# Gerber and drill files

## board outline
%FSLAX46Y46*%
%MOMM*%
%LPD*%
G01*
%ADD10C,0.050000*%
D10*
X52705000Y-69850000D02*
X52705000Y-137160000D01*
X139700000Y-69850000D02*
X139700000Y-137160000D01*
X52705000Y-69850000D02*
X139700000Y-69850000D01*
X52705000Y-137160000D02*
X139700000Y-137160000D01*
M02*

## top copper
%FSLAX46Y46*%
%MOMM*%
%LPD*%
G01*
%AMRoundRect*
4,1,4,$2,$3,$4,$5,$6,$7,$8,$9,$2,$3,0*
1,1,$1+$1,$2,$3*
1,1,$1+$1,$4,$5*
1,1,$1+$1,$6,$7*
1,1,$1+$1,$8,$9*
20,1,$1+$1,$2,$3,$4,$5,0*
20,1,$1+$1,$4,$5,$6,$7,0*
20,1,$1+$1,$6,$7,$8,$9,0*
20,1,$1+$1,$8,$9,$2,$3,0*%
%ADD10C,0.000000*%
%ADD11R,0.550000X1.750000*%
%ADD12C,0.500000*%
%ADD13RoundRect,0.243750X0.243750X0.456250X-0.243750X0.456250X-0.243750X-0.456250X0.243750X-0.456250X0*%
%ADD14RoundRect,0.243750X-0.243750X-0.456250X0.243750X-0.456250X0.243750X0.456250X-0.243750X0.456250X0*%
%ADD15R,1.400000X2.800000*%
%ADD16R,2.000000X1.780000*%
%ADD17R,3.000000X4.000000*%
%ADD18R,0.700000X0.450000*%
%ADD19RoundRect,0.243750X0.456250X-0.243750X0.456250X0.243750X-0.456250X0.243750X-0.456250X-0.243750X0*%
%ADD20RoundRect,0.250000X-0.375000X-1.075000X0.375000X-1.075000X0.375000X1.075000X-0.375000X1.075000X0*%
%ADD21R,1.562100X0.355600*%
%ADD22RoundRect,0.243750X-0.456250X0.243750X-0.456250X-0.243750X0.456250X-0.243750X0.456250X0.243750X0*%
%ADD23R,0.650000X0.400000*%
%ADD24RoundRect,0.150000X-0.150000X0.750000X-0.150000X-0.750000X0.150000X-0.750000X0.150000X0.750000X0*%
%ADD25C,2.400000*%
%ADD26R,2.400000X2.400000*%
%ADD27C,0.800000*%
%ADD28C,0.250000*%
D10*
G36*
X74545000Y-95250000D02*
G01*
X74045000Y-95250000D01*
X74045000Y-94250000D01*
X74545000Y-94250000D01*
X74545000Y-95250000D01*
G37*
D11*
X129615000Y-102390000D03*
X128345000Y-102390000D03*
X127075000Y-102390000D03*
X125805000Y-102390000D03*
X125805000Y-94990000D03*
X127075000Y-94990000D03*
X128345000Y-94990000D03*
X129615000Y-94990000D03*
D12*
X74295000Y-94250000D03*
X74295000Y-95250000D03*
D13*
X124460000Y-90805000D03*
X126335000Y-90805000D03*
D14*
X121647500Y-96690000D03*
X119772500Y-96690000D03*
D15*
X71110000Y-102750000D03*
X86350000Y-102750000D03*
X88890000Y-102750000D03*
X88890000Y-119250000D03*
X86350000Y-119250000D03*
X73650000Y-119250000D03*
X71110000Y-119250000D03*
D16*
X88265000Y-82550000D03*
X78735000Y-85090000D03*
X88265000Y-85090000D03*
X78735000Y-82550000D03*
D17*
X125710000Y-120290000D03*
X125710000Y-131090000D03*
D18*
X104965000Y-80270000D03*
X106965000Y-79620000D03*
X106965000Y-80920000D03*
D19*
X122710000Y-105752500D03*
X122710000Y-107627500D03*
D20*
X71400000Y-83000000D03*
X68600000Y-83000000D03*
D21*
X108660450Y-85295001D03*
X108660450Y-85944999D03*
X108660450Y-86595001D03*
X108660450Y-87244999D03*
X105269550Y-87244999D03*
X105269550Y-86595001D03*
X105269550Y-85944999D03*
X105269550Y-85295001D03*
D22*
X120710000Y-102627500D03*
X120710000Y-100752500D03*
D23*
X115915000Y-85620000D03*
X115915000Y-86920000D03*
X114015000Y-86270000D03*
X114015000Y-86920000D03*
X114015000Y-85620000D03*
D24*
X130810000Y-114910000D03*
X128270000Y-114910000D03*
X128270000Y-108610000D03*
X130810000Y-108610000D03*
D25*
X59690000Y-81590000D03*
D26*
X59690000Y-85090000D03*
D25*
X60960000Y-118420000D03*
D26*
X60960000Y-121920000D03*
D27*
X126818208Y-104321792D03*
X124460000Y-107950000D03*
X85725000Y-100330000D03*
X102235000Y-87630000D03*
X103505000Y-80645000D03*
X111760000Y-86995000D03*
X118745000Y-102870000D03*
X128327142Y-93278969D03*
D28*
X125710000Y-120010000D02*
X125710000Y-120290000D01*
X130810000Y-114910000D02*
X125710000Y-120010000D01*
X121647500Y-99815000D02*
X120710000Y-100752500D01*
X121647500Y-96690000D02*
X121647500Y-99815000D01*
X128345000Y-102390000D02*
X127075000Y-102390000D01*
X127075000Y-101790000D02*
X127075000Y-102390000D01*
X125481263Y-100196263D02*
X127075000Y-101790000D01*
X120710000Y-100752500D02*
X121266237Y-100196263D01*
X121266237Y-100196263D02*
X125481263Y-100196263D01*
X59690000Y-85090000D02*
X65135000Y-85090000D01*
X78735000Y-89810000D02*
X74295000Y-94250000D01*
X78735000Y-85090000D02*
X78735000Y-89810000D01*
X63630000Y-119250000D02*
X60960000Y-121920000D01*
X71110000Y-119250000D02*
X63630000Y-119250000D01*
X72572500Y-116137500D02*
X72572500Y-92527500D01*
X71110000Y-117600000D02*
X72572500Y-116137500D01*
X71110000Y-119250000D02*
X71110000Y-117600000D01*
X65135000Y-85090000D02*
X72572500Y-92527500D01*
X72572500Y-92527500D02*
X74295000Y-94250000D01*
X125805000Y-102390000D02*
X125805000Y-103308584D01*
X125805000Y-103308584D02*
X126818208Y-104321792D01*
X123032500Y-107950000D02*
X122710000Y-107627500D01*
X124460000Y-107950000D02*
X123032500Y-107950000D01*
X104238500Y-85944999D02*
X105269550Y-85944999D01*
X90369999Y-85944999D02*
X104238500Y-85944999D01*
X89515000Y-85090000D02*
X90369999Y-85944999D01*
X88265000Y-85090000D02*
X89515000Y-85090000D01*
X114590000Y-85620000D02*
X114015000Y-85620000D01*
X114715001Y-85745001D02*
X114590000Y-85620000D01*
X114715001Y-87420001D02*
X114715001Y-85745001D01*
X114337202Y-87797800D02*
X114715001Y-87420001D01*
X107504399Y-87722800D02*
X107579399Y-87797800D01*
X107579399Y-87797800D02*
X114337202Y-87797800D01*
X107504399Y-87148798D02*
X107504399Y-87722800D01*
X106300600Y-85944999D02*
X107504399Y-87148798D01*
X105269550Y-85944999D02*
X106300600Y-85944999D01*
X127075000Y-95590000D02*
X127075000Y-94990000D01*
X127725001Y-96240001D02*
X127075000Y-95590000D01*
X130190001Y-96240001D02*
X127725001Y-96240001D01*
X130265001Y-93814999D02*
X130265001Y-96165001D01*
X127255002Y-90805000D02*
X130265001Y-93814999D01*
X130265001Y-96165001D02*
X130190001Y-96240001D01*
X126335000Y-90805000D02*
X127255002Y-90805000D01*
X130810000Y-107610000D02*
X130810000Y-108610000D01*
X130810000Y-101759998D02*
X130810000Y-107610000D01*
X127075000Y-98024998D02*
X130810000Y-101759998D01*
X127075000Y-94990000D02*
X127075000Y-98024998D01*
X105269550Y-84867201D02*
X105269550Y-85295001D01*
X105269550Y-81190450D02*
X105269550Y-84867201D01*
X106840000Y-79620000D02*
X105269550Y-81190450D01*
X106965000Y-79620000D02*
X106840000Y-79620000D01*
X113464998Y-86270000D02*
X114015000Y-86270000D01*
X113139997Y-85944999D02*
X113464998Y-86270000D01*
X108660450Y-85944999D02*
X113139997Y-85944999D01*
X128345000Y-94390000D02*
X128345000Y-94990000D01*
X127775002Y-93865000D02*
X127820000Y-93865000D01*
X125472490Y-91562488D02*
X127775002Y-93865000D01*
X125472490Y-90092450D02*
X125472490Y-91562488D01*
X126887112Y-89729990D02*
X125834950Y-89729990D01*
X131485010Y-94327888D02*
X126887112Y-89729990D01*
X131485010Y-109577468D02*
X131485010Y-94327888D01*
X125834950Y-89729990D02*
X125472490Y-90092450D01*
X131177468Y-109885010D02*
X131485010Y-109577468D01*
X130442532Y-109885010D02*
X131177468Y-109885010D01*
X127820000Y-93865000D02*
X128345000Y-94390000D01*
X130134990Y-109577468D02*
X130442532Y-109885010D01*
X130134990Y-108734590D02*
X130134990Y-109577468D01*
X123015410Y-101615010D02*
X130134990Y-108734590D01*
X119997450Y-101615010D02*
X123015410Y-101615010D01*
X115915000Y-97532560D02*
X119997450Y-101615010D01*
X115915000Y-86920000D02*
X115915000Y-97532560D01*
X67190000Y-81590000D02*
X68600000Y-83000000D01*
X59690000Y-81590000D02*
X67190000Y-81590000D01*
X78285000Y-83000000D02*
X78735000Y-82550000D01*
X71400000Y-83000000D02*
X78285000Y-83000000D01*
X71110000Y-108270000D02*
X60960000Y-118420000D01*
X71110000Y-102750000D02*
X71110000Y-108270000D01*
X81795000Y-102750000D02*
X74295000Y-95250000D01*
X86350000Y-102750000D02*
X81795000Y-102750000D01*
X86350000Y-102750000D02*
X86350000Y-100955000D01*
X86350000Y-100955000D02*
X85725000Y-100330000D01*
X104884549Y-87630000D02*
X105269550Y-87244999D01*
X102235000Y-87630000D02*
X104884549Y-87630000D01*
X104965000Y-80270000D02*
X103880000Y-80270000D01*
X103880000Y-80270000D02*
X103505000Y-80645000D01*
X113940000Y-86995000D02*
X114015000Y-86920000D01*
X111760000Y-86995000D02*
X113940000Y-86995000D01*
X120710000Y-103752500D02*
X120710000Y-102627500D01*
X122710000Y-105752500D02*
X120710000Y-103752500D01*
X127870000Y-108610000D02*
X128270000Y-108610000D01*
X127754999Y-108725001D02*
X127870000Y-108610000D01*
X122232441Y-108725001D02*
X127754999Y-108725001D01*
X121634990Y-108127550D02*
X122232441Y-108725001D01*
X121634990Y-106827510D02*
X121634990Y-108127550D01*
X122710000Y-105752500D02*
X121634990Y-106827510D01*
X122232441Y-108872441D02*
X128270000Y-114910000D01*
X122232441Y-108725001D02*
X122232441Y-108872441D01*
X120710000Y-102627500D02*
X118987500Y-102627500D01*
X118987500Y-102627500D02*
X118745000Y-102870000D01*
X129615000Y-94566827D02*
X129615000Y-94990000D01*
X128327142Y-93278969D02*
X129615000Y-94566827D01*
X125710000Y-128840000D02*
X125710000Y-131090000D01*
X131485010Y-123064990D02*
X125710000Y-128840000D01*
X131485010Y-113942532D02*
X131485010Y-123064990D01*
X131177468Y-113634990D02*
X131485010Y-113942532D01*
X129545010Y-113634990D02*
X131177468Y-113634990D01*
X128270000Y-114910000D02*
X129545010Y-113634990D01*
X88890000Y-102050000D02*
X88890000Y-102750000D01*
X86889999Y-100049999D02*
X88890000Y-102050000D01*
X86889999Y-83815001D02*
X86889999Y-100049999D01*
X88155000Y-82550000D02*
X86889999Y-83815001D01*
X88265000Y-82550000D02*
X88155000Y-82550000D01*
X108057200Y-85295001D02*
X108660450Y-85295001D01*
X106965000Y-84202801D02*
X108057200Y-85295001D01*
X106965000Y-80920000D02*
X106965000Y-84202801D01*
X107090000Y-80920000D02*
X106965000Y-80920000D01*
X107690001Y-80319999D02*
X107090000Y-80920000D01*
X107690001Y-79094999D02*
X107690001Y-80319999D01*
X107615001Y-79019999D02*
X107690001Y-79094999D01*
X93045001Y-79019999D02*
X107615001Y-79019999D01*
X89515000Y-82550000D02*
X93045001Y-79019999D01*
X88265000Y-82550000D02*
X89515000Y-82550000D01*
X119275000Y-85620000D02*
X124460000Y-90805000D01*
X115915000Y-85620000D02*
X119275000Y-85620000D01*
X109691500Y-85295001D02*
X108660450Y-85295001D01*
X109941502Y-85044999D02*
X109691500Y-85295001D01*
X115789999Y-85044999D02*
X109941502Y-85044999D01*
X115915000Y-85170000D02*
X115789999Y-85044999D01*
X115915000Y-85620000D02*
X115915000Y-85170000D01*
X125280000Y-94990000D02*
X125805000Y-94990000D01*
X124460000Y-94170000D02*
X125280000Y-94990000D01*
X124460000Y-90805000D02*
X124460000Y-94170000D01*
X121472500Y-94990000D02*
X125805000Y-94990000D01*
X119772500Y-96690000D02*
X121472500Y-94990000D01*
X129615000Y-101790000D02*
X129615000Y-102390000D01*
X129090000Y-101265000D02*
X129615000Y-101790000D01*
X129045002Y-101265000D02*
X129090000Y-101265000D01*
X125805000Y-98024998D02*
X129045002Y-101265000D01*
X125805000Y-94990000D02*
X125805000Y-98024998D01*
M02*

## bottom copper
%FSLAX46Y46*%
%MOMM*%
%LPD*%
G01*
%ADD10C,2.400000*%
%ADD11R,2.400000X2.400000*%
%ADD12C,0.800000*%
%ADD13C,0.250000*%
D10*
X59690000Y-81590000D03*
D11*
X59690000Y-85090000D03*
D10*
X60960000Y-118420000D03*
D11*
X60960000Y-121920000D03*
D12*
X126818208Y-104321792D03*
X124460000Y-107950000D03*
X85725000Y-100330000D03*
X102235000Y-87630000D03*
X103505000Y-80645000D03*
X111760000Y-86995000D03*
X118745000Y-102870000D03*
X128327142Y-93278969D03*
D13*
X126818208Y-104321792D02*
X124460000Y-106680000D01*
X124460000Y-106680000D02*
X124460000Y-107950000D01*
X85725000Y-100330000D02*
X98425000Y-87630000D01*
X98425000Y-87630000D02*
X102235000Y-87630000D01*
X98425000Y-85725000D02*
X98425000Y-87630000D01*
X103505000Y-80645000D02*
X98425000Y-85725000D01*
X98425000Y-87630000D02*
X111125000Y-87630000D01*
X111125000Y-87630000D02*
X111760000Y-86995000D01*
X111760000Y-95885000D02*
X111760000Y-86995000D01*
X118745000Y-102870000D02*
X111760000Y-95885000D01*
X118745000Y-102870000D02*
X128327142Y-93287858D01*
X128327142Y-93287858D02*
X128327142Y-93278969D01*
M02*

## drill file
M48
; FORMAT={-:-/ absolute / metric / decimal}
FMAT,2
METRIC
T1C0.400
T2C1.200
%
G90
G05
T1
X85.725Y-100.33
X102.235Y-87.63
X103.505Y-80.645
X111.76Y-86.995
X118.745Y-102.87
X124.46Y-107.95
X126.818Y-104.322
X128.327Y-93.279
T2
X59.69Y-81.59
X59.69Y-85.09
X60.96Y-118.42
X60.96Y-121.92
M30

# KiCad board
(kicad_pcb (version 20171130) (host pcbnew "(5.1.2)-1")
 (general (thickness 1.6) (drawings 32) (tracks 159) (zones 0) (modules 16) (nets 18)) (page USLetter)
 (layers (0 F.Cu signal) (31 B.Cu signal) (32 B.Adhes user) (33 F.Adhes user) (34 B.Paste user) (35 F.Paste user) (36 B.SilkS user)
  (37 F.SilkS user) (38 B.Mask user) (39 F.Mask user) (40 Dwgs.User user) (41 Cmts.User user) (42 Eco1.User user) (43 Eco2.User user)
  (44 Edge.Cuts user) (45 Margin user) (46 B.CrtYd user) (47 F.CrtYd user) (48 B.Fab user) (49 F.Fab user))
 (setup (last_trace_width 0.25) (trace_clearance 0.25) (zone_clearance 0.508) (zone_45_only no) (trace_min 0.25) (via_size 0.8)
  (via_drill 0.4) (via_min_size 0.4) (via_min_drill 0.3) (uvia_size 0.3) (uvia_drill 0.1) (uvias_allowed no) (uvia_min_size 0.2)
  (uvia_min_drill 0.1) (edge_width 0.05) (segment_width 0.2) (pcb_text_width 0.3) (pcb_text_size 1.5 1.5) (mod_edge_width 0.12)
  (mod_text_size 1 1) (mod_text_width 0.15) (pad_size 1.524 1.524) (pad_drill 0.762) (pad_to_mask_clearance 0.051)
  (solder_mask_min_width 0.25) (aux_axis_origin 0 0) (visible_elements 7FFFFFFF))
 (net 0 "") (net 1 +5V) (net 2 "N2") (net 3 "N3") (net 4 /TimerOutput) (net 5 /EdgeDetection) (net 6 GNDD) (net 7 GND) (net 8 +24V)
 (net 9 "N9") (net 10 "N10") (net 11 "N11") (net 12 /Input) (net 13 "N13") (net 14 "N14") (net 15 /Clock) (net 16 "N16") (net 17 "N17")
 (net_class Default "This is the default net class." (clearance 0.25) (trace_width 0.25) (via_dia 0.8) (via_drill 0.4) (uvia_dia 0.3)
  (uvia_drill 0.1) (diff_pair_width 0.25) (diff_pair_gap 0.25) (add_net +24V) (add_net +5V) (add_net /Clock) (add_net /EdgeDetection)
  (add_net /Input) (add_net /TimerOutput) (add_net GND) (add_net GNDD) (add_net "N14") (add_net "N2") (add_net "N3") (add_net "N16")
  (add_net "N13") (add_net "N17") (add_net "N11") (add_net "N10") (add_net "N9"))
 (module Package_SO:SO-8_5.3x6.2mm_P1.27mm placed (layer F.Cu) (at 127.71 98.69 270)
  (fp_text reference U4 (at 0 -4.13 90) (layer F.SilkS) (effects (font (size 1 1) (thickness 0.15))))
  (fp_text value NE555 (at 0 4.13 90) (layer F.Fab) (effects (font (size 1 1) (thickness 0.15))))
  (pad 8 smd rect (at 3.7 -1.905 270) (size 1.75 0.55) (layers F.Cu F.Paste F.Mask) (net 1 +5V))
  (pad 7 smd rect (at 3.7 -0.635 270) (size 1.75 0.55) (layers F.Cu F.Paste F.Mask) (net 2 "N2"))
  (pad 6 smd rect (at 3.7 0.635 270) (size 1.75 0.55) (layers F.Cu F.Paste F.Mask) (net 2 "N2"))
  (pad 5 smd rect (at 3.7 1.905 270) (size 1.75 0.55) (layers F.Cu F.Paste F.Mask) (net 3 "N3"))
  (pad 4 smd rect (at -3.7 1.905 270) (size 1.75 0.55) (layers F.Cu F.Paste F.Mask) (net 1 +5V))
  (pad 3 smd rect (at -3.7 0.635 270) (size 1.75 0.55) (layers F.Cu F.Paste F.Mask) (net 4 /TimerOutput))
  (pad 2 smd rect (at -3.7 -0.635 270) (size 1.75 0.55) (layers F.Cu F.Paste F.Mask) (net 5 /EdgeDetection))
  (pad 1 smd rect (at -3.7 -1.905 270) (size 1.75 0.55) (layers F.Cu F.Paste F.Mask) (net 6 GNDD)))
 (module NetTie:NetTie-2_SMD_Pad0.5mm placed (layer F.Cu) (at 74.295 94.75 90)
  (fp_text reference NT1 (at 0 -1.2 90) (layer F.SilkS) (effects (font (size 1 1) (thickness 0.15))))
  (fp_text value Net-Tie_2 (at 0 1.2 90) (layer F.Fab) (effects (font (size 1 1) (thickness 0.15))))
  (fp_poly (pts (xy -0.5 -0.25) (xy 0.5 -0.25) (xy 0.5 0.25) (xy -0.5 0.25)) (layer F.Cu) (width 0))
  (pad 2 smd circle (at 0.5 0 90) (size 0.5 0.5) (layers F.Cu) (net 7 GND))
  (pad 1 smd circle (at -0.5 0 90) (size 0.5 0.5) (layers F.Cu) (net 6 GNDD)))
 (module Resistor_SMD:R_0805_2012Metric (layer F.Cu) (at 125.3975 90.805 180)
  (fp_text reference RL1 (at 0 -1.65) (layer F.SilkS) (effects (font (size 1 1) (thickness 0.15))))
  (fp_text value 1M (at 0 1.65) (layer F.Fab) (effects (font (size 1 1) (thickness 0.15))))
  (pad 2 smd roundrect (at 0.9375 0 180) (size 0.975 1.4) (layers F.Cu F.Paste F.Mask) (roundrect_rratio 0.25) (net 1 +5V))
  (pad 1 smd roundrect (at -0.9375 0 180) (size 0.975 1.4) (layers F.Cu F.Paste F.Mask) (roundrect_rratio 0.25) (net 4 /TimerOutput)))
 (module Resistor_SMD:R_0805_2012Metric (layer F.Cu) (at 120.71 96.69)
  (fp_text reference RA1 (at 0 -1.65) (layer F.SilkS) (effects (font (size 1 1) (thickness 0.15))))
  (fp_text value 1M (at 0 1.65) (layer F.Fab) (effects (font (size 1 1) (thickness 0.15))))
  (pad 2 smd roundrect (at 0.9375 0) (size 0.975 1.4) (layers F.Cu F.Paste F.Mask) (roundrect_rratio 0.25) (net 2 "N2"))
  (pad 1 smd roundrect (at -0.9375 0) (size 0.975 1.4) (layers F.Cu F.Paste F.Mask) (roundrect_rratio 0.25) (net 1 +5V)))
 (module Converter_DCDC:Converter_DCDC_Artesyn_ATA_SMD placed (layer F.Cu) (at 80 111 90)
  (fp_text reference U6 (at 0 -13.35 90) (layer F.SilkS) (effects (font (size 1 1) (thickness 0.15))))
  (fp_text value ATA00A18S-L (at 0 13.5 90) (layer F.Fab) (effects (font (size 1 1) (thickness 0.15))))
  (pad 16 smd rect (at 8.25 -8.89 90) (size 2.8 1.4) (layers F.Cu F.Paste F.Mask) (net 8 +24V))
  (pad 10 smd rect (at 8.25 6.35 90) (size 2.8 1.4) (layers F.Cu F.Paste F.Mask) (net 6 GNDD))
  (pad 9 smd rect (at 8.25 8.89 90) (size 2.8 1.4) (layers F.Cu F.Paste F.Mask) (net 1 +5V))
  (pad 8 smd rect (at -8.25 8.89 90) (size 2.8 1.4) (layers F.Cu F.Paste F.Mask) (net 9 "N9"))
  (pad 7 smd rect (at -8.25 6.35 90) (size 2.8 1.4) (layers F.Cu F.Paste F.Mask) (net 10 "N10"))
  (pad 2 smd rect (at -8.25 -6.35 90) (size 2.8 1.4) (layers F.Cu F.Paste F.Mask) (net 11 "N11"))
  (pad 1 smd rect (at -8.25 -8.89 90) (size 2.8 1.4) (layers F.Cu F.Paste F.Mask) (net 7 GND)))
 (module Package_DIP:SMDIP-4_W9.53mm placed (layer F.Cu) (at 83.5 83.82)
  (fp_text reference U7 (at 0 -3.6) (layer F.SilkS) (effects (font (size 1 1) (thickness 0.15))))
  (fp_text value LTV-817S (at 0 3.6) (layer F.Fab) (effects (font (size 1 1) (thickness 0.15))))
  (pad 4 smd rect (at 4.765 -1.27) (size 2 1.78) (layers F.Cu F.Paste F.Mask) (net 1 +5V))
  (pad 2 smd rect (at -4.765 1.27) (size 2 1.78) (layers F.Cu F.Paste F.Mask) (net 7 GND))
  (pad 3 smd rect (at 4.765 1.27) (size 2 1.78) (layers F.Cu F.Paste F.Mask) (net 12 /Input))
  (pad 1 smd rect (at -4.765 -1.27) (size 2 1.78) (layers F.Cu F.Paste F.Mask) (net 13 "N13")))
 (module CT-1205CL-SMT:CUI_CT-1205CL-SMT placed (layer F.Cu) (at 125.71 125.69 90)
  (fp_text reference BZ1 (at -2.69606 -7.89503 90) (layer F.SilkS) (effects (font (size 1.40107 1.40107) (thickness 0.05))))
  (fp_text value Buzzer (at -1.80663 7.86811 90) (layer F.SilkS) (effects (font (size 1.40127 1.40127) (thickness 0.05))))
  (pad 1 smd rect (at 5.4 0 90) (size 4 3) (layers F.Cu F.Paste F.Mask) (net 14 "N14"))
  (pad 2 smd rect (at -5.4 0 90) (size 4 3) (layers F.Cu F.Paste F.Mask) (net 6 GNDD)))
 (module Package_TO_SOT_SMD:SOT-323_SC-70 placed (layer F.Cu) (at 105.965 80.27 180)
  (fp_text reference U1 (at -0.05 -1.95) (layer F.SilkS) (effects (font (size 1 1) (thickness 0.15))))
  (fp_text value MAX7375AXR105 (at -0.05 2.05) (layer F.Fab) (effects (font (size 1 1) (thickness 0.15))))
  (pad 3 smd rect (at 1 0 90) (size 0.45 0.7) (layers F.Cu F.Paste F.Mask) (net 6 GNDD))
  (pad 2 smd rect (at -1 0.65 90) (size 0.45 0.7) (layers F.Cu F.Paste F.Mask) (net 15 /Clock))
  (pad 1 smd rect (at -1 -0.65 90) (size 0.45 0.7) (layers F.Cu F.Paste F.Mask) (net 1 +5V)))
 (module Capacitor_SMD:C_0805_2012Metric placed (layer F.Cu) (at 122.71 106.69 90)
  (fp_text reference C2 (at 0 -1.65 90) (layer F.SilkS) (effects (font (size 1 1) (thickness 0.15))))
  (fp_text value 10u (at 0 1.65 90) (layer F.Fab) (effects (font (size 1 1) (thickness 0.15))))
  (pad 2 smd roundrect (at 0.9375 0 90) (size 0.975 1.4) (layers F.Cu F.Paste F.Mask) (roundrect_rratio 0.25) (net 6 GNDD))
  (pad 1 smd roundrect (at -0.9375 0 90) (size 0.975 1.4) (layers F.Cu F.Paste F.Mask) (roundrect_rratio 0.25) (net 3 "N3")))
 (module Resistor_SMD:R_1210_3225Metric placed (layer F.Cu) (at 70 83)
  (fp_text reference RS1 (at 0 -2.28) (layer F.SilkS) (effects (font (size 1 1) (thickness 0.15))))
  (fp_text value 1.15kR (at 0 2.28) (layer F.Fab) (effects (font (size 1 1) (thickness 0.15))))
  (pad 2 smd roundrect (at 1.4 0) (size 1.25 2.65) (layers F.Cu F.Paste F.Mask) (roundrect_rratio 0.2) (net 13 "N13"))
  (pad 1 smd roundrect (at -1.4 0) (size 1.25 2.65) (layers F.Cu F.Paste F.Mask) (roundrect_rratio 0.2) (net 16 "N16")))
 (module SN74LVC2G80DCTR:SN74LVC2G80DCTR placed (layer F.Cu) (at 106.965 86.27)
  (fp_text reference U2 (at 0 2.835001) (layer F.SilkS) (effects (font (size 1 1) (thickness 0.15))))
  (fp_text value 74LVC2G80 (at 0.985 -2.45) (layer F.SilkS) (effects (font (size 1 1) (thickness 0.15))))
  (pad 8 smd rect (at 1.69545 -0.974999) (size 1.5621 0.3556) (layers F.Cu F.Paste F.Mask) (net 1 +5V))
  (pad 7 smd rect (at 1.69545 -0.325001) (size 1.5621 0.3556) (layers F.Cu F.Paste F.Mask) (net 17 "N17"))
  (pad 6 smd rect (at 1.69545 0.325001) (size 1.5621 0.3556) (layers F.Cu F.Paste F.Mask))
  (pad 5 smd rect (at 1.69545 0.974999) (size 1.5621 0.3556) (layers F.Cu F.Paste F.Mask))
  (pad 4 smd rect (at -1.69545 0.974999) (size 1.5621 0.3556) (layers F.Cu F.Paste F.Mask) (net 6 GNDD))
  (pad 3 smd rect (at -1.69545 0.325001) (size 1.5621 0.3556) (layers F.Cu F.Paste F.Mask))
  (pad 2 smd rect (at -1.69545 -0.325001) (size 1.5621 0.3556) (layers F.Cu F.Paste F.Mask) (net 12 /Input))
  (pad 1 smd rect (at -1.69545 -0.974999) (size 1.5621 0.3556) (layers F.Cu F.Paste F.Mask) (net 15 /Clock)))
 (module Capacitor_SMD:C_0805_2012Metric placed (layer F.Cu) (at 120.71 101.69 270)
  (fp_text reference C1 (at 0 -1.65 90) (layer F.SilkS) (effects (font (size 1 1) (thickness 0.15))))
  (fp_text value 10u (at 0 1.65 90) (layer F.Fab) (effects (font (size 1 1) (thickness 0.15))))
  (pad 2 smd roundrect (at 0.9375 0 270) (size 0.975 1.4) (layers F.Cu F.Paste F.Mask) (roundrect_rratio 0.25) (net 6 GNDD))
  (pad 1 smd roundrect (at -0.9375 0 270) (size 0.975 1.4) (layers F.Cu F.Paste F.Mask) (roundrect_rratio 0.25) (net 2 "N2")))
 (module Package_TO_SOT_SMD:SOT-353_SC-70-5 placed (layer F.Cu) (at 114.965 86.27)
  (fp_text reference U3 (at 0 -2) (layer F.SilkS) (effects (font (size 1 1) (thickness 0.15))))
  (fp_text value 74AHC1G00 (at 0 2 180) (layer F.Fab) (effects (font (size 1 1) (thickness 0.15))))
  (pad 5 smd rect (at 0.95 -0.65) (size 0.65 0.4) (layers F.Cu F.Paste F.Mask) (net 1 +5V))
  (pad 4 smd rect (at 0.95 0.65) (size 0.65 0.4) (layers F.Cu F.Paste F.Mask) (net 5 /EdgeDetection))
  (pad 2 smd rect (at -0.95 0) (size 0.65 0.4) (layers F.Cu F.Paste F.Mask) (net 17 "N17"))
  (pad 3 smd rect (at -0.95 0.65) (size 0.65 0.4) (layers F.Cu F.Paste F.Mask) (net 6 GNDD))
  (pad 1 smd rect (at -0.95 -0.65) (size 0.65 0.4) (layers F.Cu F.Paste F.Mask) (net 12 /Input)))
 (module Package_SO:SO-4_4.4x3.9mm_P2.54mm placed (layer F.Cu) (at 129.54 111.76 270)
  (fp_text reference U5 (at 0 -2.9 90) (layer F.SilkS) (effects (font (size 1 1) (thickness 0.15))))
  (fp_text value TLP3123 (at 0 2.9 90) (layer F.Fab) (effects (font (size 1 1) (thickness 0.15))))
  (pad 4 smd roundrect (at 3.15 -1.27 270) (size 1.8 0.6) (layers F.Cu F.Paste F.Mask) (roundrect_rratio 0.25) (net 14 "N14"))
  (pad 3 smd roundrect (at 3.15 1.27 270) (size 1.8 0.6) (layers F.Cu F.Paste F.Mask) (roundrect_rratio 0.25) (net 6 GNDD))
  (pad 2 smd roundrect (at -3.15 1.27 270) (size 1.8 0.6) (layers F.Cu F.Paste F.Mask) (roundrect_rratio 0.25) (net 6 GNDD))
  (pad 1 smd roundrect (at -3.15 -1.27 270) (size 1.8 0.6) (layers F.Cu F.Paste F.Mask) (roundrect_rratio 0.25) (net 4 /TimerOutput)))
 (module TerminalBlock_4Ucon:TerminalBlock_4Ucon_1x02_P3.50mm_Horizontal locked (layer F.Cu) (at 59.69 85.09 90)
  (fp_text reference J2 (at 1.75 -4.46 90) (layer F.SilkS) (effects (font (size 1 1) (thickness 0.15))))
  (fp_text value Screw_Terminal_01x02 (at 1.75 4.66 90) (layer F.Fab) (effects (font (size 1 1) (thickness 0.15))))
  (pad 2 thru_hole circle (at 3.5 0 90) (size 2.4 2.4) (drill 1.2) (layers *.Cu *.Mask) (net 16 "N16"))
  (pad 1 thru_hole rect (at 0 0 90) (size 2.4 2.4) (drill 1.2) (layers *.Cu *.Mask) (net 7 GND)))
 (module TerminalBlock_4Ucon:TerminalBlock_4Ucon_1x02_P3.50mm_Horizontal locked (layer F.Cu) (at 60.96 121.92 90)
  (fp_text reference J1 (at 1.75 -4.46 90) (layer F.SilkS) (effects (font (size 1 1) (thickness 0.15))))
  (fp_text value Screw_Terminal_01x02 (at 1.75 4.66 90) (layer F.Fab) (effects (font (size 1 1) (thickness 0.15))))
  (pad 2 thru_hole circle (at 3.5 0 90) (size 2.4 2.4) (drill 1.2) (layers *.Cu *.Mask) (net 8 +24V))
  (pad 1 thru_hole rect (at 0 0 90) (size 2.4 2.4) (drill 1.2) (layers *.Cu *.Mask) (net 7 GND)))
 (gr_line (start 52.705 69.85) (end 52.705 137.16) (layer Edge.Cuts) (width 0.05))
 (gr_line (start 139.7 69.85) (end 139.7 137.16) (layer Edge.Cuts) (width 0.05))
 (gr_line (start 52.705 69.85) (end 139.7 69.85) (layer Edge.Cuts) (width 0.05))
 (gr_line (start 52.705 137.16) (end 139.7 137.16) (layer Edge.Cuts) (width 0.05))
 (segment (start 125.71 120.01) (end 125.71 120.29) (width 0.25) (layer F.Cu) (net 14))
 (segment (start 130.81 114.91) (end 125.71 120.01) (width 0.25) (layer F.Cu) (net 14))
 (segment (start 121.6475 99.815) (end 120.71 100.7525) (width 0.25) (layer F.Cu) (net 2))
 (segment (start 121.6475 96.69) (end 121.6475 99.815) (width 0.25) (layer F.Cu) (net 2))
 (segment (start 128.345 102.39) (end 127.075 102.39) (width 0.25) (layer F.Cu) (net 2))
 (segment (start 127.075 101.79) (end 127.075 102.39) (width 0.25) (layer F.Cu) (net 2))
 (segment (start 125.481263 100.196263) (end 127.075 101.79) (width 0.25) (layer F.Cu) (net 2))
 (segment (start 120.71 100.7525) (end 121.266237 100.196263) (width 0.25) (layer F.Cu) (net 2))
 (segment (start 121.266237 100.196263) (end 125.481263 100.196263) (width 0.25) (layer F.Cu) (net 2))
 (segment (start 59.69 85.09) (end 65.135 85.09) (width 0.25) (layer F.Cu) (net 7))
 (segment (start 78.735 89.81) (end 74.295 94.25) (width 0.25) (layer F.Cu) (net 7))
 (segment (start 78.735 85.09) (end 78.735 89.81) (width 0.25) (layer F.Cu) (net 7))
 (segment (start 63.63 119.25) (end 60.96 121.92) (width 0.25) (layer F.Cu) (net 7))
 (segment (start 71.11 119.25) (end 63.63 119.25) (width 0.25) (layer F.Cu) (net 7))
 (segment (start 72.5725 116.1375) (end 72.5725 92.5275) (width 0.25) (layer F.Cu) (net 7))
 (segment (start 71.11 117.6) (end 72.5725 116.1375) (width 0.25) (layer F.Cu) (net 7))
 (segment (start 71.11 119.25) (end 71.11 117.6) (width 0.25) (layer F.Cu) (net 7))
 (segment (start 65.135 85.09) (end 72.5725 92.5275) (width 0.25) (layer F.Cu) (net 7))
 (segment (start 72.5725 92.5275) (end 74.295 94.25) (width 0.25) (layer F.Cu) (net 7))
 (via (at 126.818208 104.321792) (size 0.8) (drill 0.4) (layers F.Cu B.Cu) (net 3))
 (segment (start 125.805 102.39) (end 125.805 103.308584) (width 0.25) (layer F.Cu) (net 3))
 (segment (start 125.805 103.308584) (end 126.818208 104.321792) (width 0.25) (layer F.Cu) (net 3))
 (via (at 124.46 107.95) (size 0.8) (drill 0.4) (layers F.Cu B.Cu) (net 3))
 (segment (start 126.818208 104.321792) (end 124.46 106.68) (width 0.25) (layer B.Cu) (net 3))
 (segment (start 124.46 106.68) (end 124.46 107.95) (width 0.25) (layer B.Cu) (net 3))
 (segment (start 123.0325 107.95) (end 122.71 107.6275) (width 0.25) (layer F.Cu) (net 3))
 (segment (start 124.46 107.95) (end 123.0325 107.95) (width 0.25) (layer F.Cu) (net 3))
 (segment (start 104.2385 85.944999) (end 105.26955 85.944999) (width 0.25) (layer F.Cu) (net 12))
 (segment (start 90.369999 85.944999) (end 104.2385 85.944999) (width 0.25) (layer F.Cu) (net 12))
 (segment (start 89.515 85.09) (end 90.369999 85.944999) (width 0.25) (layer F.Cu) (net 12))
 (segment (start 88.265 85.09) (end 89.515 85.09) (width 0.25) (layer F.Cu) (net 12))
 (segment (start 114.59 85.62) (end 114.015 85.62) (width 0.25) (layer F.Cu) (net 12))
 (segment (start 114.715001 85.745001) (end 114.59 85.62) (width 0.25) (layer F.Cu) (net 12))
 (segment (start 114.715001 87.420001) (end 114.715001 85.745001) (width 0.25) (layer F.Cu) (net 12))
 (segment (start 114.337202 87.7978) (end 114.715001 87.420001) (width 0.25) (layer F.Cu) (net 12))
 (segment (start 107.504399 87.7228) (end 107.579399 87.7978) (width 0.25) (layer F.Cu) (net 12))
 (segment (start 107.579399 87.7978) (end 114.337202 87.7978) (width 0.25) (layer F.Cu) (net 12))
 (segment (start 107.504399 87.148798) (end 107.504399 87.7228) (width 0.25) (layer F.Cu) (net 12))
 (segment (start 106.3006 85.944999) (end 107.504399 87.148798) (width 0.25) (layer F.Cu) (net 12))
 (segment (start 105.26955 85.944999) (end 106.3006 85.944999) (width 0.25) (layer F.Cu) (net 12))
 (segment (start 127.075 95.59) (end 127.075 94.99) (width 0.25) (layer F.Cu) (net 4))
 (segment (start 127.725001 96.240001) (end 127.075 95.59) (width 0.25) (layer F.Cu) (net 4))
 (segment (start 130.190001 96.240001) (end 127.725001 96.240001) (width 0.25) (layer F.Cu) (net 4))
 (segment (start 130.265001 93.814999) (end 130.265001 96.165001) (width 0.25) (layer F.Cu) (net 4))
 (segment (start 127.255002 90.805) (end 130.265001 93.814999) (width 0.25) (layer F.Cu) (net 4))
 (segment (start 130.265001 96.165001) (end 130.190001 96.240001) (width 0.25) (layer F.Cu) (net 4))
 (segment (start 126.335 90.805) (end 127.255002 90.805) (width 0.25) (layer F.Cu) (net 4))
 (segment (start 130.81 107.61) (end 130.81 108.61) (width 0.25) (layer F.Cu) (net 4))
 (segment (start 130.81 101.759998) (end 130.81 107.61) (width 0.25) (layer F.Cu) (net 4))
 (segment (start 127.075 98.024998) (end 130.81 101.759998) (width 0.25) (layer F.Cu) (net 4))
 (segment (start 127.075 94.99) (end 127.075 98.024998) (width 0.25) (layer F.Cu) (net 4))
 (segment (start 105.26955 84.867201) (end 105.26955 85.295001) (width 0.25) (layer F.Cu) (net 15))
 (segment (start 105.26955 81.19045) (end 105.26955 84.867201) (width 0.25) (layer F.Cu) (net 15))
 (segment (start 106.84 79.62) (end 105.26955 81.19045) (width 0.25) (layer F.Cu) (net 15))
 (segment (start 106.965 79.62) (end 106.84 79.62) (width 0.25) (layer F.Cu) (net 15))
 (segment (start 113.464998 86.27) (end 114.015 86.27) (width 0.25) (layer F.Cu) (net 17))
 (segment (start 113.139997 85.944999) (end 113.464998 86.27) (width 0.25) (layer F.Cu) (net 17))
 (segment (start 108.66045 85.944999) (end 113.139997 85.944999) (width 0.25) (layer F.Cu) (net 17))
 (segment (start 128.345 94.39) (end 128.345 94.99) (width 0.25) (layer F.Cu) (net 5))
 (segment (start 127.775002 93.865) (end 127.82 93.865) (width 0.25) (layer F.Cu) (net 5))
 (segment (start 125.47249 91.562488) (end 127.775002 93.865) (width 0.25) (layer F.Cu) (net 5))
 (segment (start 125.47249 90.09245) (end 125.47249 91.562488) (width 0.25) (layer F.Cu) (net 5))
 (segment (start 126.887112 89.72999) (end 125.83495 89.72999) (width 0.25) (layer F.Cu) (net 5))
 (segment (start 131.48501 94.327888) (end 126.887112 89.72999) (width 0.25) (layer F.Cu) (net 5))
 (segment (start 131.48501 109.577468) (end 131.48501 94.327888) (width 0.25) (layer F.Cu) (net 5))
 (segment (start 125.83495 89.72999) (end 125.47249 90.09245) (width 0.25) (layer F.Cu) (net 5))
 (segment (start 131.177468 109.88501) (end 131.48501 109.577468) (width 0.25) (layer F.Cu) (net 5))
 (segment (start 130.442532 109.88501) (end 131.177468 109.88501) (width 0.25) (layer F.Cu) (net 5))
 (segment (start 127.82 93.865) (end 128.345 94.39) (width 0.25) (layer F.Cu) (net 5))
 (segment (start 130.13499 109.577468) (end 130.442532 109.88501) (width 0.25) (layer F.Cu) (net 5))
 (segment (start 130.13499 108.73459) (end 130.13499 109.577468) (width 0.25) (layer F.Cu) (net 5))
 (segment (start 123.01541 101.61501) (end 130.13499 108.73459) (width 0.25) (layer F.Cu) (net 5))
 (segment (start 119.99745 101.61501) (end 123.01541 101.61501) (width 0.25) (layer F.Cu) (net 5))
 (segment (start 115.915 97.53256) (end 119.99745 101.61501) (width 0.25) (layer F.Cu) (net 5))
 (segment (start 115.915 86.92) (end 115.915 97.53256) (width 0.25) (layer F.Cu) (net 5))
 (segment (start 67.19 81.59) (end 68.6 83) (width 0.25) (layer F.Cu) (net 16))
 (segment (start 59.69 81.59) (end 67.19 81.59) (width 0.25) (layer F.Cu) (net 16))
 (segment (start 78.285 83) (end 78.735 82.55) (width 0.25) (layer F.Cu) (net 13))
 (segment (start 71.4 83) (end 78.285 83) (width 0.25) (layer F.Cu) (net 13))
 (segment (start 71.11 108.27) (end 60.96 118.42) (width 0.25) (layer F.Cu) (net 8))
 (segment (start 71.11 102.75) (end 71.11 108.27) (width 0.25) (layer F.Cu) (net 8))
 (segment (start 81.795 102.75) (end 74.295 95.25) (width 0.25) (layer F.Cu) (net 6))
 (segment (start 86.35 102.75) (end 81.795 102.75) (width 0.25) (layer F.Cu) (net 6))
 (via (at 85.725 100.33) (size 0.8) (drill 0.4) (layers F.Cu B.Cu) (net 6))
 (segment (start 86.35 102.75) (end 86.35 100.955) (width 0.25) (layer F.Cu) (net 6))
 (segment (start 86.35 100.955) (end 85.725 100.33) (width 0.25) (layer F.Cu) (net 6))
 (via (at 102.235 87.63) (size 0.8) (drill 0.4) (layers F.Cu B.Cu) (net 6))
 (segment (start 85.725 100.33) (end 98.425 87.63) (width 0.25) (layer B.Cu) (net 6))
 (segment (start 98.425 87.63) (end 102.235 87.63) (width 0.25) (layer B.Cu) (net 6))
 (segment (start 104.884549 87.63) (end 105.26955 87.244999) (width 0.25) (layer F.Cu) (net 6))
 (segment (start 102.235 87.63) (end 104.884549 87.63) (width 0.25) (layer F.Cu) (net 6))
 (via (at 103.505 80.645) (size 0.8) (drill 0.4) (layers F.Cu B.Cu) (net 6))
 (segment (start 104.965 80.27) (end 103.88 80.27) (width 0.25) (layer F.Cu) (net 6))
 (segment (start 103.88 80.27) (end 103.505 80.645) (width 0.25) (layer F.Cu) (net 6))
 (segment (start 98.425 85.725) (end 98.425 87.63) (width 0.25) (layer B.Cu) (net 6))
 (segment (start 103.505 80.645) (end 98.425 85.725) (width 0.25) (layer B.Cu) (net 6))
 (via (at 111.76 86.995) (size 0.8) (drill 0.4) (layers F.Cu B.Cu) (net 6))
 (segment (start 98.425 87.63) (end 111.125 87.63) (width 0.25) (layer B.Cu) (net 6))
 (segment (start 111.125 87.63) (end 111.76 86.995) (width 0.25) (layer B.Cu) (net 6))
 (segment (start 113.94 86.995) (end 114.015 86.92) (width 0.25) (layer F.Cu) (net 6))
 (segment (start 111.76 86.995) (end 113.94 86.995) (width 0.25) (layer F.Cu) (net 6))
 (segment (start 120.71 103.7525) (end 120.71 102.6275) (width 0.25) (layer F.Cu) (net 6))
 (segment (start 122.71 105.7525) (end 120.71 103.7525) (width 0.25) (layer F.Cu) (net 6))
 (segment (start 127.87 108.61) (end 128.27 108.61) (width 0.25) (layer F.Cu) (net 6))
 (segment (start 127.754999 108.725001) (end 127.87 108.61) (width 0.25) (layer F.Cu) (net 6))
 (segment (start 122.232441 108.725001) (end 127.754999 108.725001) (width 0.25) (layer F.Cu) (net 6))
 (segment (start 121.63499 108.12755) (end 122.232441 108.725001) (width 0.25) (layer F.Cu) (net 6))
 (segment (start 121.63499 106.82751) (end 121.63499 108.12755) (width 0.25) (layer F.Cu) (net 6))
 (segment (start 122.71 105.7525) (end 121.63499 106.82751) (width 0.25) (layer F.Cu) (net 6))
 (segment (start 122.232441 108.872441) (end 128.27 114.91) (width 0.25) (layer F.Cu) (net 6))
 (segment (start 122.232441 108.725001) (end 122.232441 108.872441) (width 0.25) (layer F.Cu) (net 6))
 (via (at 118.745 102.87) (size 0.8) (drill 0.4) (layers F.Cu B.Cu) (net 6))
 (segment (start 120.71 102.6275) (end 118.9875 102.6275) (width 0.25) (layer F.Cu) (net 6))
 (segment (start 118.9875 102.6275) (end 118.745 102.87) (width 0.25) (layer F.Cu) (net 6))
 (segment (start 111.76 95.885) (end 111.76 86.995) (width 0.25) (layer B.Cu) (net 6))
 (segment (start 118.745 102.87) (end 111.76 95.885) (width 0.25) (layer B.Cu) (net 6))
 (via (at 128.327142 93.278969) (size 0.8) (drill 0.4) (layers F.Cu B.Cu) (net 6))
 (segment (start 118.745 102.87) (end 128.327142 93.287858) (width 0.25) (layer B.Cu) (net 6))
 (segment (start 128.327142 93.287858) (end 128.327142 93.278969) (width 0.25) (layer B.Cu) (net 6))
 (segment (start 129.615 94.566827) (end 129.615 94.99) (width 0.25) (layer F.Cu) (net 6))
 (segment (start 128.327142 93.278969) (end 129.615 94.566827) (width 0.25) (layer F.Cu) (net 6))
 (segment (start 125.71 128.84) (end 125.71 131.09) (width 0.25) (layer F.Cu) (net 6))
 (segment (start 131.48501 123.06499) (end 125.71 128.84) (width 0.25) (layer F.Cu) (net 6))
 (segment (start 131.48501 113.942532) (end 131.48501 123.06499) (width 0.25) (layer F.Cu) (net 6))
 (segment (start 131.177468 113.63499) (end 131.48501 113.942532) (width 0.25) (layer F.Cu) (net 6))
 (segment (start 129.54501 113.63499) (end 131.177468 113.63499) (width 0.25) (layer F.Cu) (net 6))
 (segment (start 128.27 114.91) (end 129.54501 113.63499) (width 0.25) (layer F.Cu) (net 6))
 (segment (start 88.89 102.05) (end 88.89 102.75) (width 0.25) (layer F.Cu) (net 1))
 (segment (start 86.889999 100.049999) (end 88.89 102.05) (width 0.25) (layer F.Cu) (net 1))
 (segment (start 86.889999 83.815001) (end 86.889999 100.049999) (width 0.25) (layer F.Cu) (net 1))
 (segment (start 88.155 82.55) (end 86.889999 83.815001) (width 0.25) (layer F.Cu) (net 1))
 (segment (start 88.265 82.55) (end 88.155 82.55) (width 0.25) (layer F.Cu) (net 1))
 (segment (start 108.0572 85.295001) (end 108.66045 85.295001) (width 0.25) (layer F.Cu) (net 1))
 (segment (start 106.965 84.202801) (end 108.0572 85.295001) (width 0.25) (layer F.Cu) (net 1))
 (segment (start 106.965 80.92) (end 106.965 84.202801) (width 0.25) (layer F.Cu) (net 1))
 (segment (start 107.09 80.92) (end 106.965 80.92) (width 0.25) (layer F.Cu) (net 1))
 (segment (start 107.690001 80.319999) (end 107.09 80.92) (width 0.25) (layer F.Cu) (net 1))
 (segment (start 107.690001 79.094999) (end 107.690001 80.319999) (width 0.25) (layer F.Cu) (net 1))
 (segment (start 107.615001 79.019999) (end 107.690001 79.094999) (width 0.25) (layer F.Cu) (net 1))
 (segment (start 93.045001 79.019999) (end 107.615001 79.019999) (width 0.25) (layer F.Cu) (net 1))
 (segment (start 89.515 82.55) (end 93.045001 79.019999) (width 0.25) (layer F.Cu) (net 1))
 (segment (start 88.265 82.55) (end 89.515 82.55) (width 0.25) (layer F.Cu) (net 1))
 (segment (start 119.275 85.62) (end 124.46 90.805) (width 0.25) (layer F.Cu) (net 1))
 (segment (start 115.915 85.62) (end 119.275 85.62) (width 0.25) (layer F.Cu) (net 1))
 (segment (start 109.6915 85.295001) (end 108.66045 85.295001) (width 0.25) (layer F.Cu) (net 1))
 (segment (start 109.941502 85.044999) (end 109.6915 85.295001) (width 0.25) (layer F.Cu) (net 1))
 (segment (start 115.789999 85.044999) (end 109.941502 85.044999) (width 0.25) (layer F.Cu) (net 1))
 (segment (start 115.915 85.17) (end 115.789999 85.044999) (width 0.25) (layer F.Cu) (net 1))
 (segment (start 115.915 85.62) (end 115.915 85.17) (width 0.25) (layer F.Cu) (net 1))
 (segment (start 125.28 94.99) (end 125.805 94.99) (width 0.25) (layer F.Cu) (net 1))
 (segment (start 124.46 94.17) (end 125.28 94.99) (width 0.25) (layer F.Cu) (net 1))
 (segment (start 124.46 90.805) (end 124.46 94.17) (width 0.25) (layer F.Cu) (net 1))
 (segment (start 121.4725 94.99) (end 125.805 94.99) (width 0.25) (layer F.Cu) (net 1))
 (segment (start 119.7725 96.69) (end 121.4725 94.99) (width 0.25) (layer F.Cu) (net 1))
 (segment (start 129.615 101.79) (end 129.615 102.39) (width 0.25) (layer F.Cu) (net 1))
 (segment (start 129.09 101.265) (end 129.615 101.79) (width 0.25) (layer F.Cu) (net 1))
 (segment (start 129.045002 101.265) (end 129.09 101.265) (width 0.25) (layer F.Cu) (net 1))
 (segment (start 125.805 98.024998) (end 129.045002 101.265) (width 0.25) (layer F.Cu) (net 1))
 (segment (start 125.805 94.99) (end 125.805 98.024998) (width 0.25) (layer F.Cu) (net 1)))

